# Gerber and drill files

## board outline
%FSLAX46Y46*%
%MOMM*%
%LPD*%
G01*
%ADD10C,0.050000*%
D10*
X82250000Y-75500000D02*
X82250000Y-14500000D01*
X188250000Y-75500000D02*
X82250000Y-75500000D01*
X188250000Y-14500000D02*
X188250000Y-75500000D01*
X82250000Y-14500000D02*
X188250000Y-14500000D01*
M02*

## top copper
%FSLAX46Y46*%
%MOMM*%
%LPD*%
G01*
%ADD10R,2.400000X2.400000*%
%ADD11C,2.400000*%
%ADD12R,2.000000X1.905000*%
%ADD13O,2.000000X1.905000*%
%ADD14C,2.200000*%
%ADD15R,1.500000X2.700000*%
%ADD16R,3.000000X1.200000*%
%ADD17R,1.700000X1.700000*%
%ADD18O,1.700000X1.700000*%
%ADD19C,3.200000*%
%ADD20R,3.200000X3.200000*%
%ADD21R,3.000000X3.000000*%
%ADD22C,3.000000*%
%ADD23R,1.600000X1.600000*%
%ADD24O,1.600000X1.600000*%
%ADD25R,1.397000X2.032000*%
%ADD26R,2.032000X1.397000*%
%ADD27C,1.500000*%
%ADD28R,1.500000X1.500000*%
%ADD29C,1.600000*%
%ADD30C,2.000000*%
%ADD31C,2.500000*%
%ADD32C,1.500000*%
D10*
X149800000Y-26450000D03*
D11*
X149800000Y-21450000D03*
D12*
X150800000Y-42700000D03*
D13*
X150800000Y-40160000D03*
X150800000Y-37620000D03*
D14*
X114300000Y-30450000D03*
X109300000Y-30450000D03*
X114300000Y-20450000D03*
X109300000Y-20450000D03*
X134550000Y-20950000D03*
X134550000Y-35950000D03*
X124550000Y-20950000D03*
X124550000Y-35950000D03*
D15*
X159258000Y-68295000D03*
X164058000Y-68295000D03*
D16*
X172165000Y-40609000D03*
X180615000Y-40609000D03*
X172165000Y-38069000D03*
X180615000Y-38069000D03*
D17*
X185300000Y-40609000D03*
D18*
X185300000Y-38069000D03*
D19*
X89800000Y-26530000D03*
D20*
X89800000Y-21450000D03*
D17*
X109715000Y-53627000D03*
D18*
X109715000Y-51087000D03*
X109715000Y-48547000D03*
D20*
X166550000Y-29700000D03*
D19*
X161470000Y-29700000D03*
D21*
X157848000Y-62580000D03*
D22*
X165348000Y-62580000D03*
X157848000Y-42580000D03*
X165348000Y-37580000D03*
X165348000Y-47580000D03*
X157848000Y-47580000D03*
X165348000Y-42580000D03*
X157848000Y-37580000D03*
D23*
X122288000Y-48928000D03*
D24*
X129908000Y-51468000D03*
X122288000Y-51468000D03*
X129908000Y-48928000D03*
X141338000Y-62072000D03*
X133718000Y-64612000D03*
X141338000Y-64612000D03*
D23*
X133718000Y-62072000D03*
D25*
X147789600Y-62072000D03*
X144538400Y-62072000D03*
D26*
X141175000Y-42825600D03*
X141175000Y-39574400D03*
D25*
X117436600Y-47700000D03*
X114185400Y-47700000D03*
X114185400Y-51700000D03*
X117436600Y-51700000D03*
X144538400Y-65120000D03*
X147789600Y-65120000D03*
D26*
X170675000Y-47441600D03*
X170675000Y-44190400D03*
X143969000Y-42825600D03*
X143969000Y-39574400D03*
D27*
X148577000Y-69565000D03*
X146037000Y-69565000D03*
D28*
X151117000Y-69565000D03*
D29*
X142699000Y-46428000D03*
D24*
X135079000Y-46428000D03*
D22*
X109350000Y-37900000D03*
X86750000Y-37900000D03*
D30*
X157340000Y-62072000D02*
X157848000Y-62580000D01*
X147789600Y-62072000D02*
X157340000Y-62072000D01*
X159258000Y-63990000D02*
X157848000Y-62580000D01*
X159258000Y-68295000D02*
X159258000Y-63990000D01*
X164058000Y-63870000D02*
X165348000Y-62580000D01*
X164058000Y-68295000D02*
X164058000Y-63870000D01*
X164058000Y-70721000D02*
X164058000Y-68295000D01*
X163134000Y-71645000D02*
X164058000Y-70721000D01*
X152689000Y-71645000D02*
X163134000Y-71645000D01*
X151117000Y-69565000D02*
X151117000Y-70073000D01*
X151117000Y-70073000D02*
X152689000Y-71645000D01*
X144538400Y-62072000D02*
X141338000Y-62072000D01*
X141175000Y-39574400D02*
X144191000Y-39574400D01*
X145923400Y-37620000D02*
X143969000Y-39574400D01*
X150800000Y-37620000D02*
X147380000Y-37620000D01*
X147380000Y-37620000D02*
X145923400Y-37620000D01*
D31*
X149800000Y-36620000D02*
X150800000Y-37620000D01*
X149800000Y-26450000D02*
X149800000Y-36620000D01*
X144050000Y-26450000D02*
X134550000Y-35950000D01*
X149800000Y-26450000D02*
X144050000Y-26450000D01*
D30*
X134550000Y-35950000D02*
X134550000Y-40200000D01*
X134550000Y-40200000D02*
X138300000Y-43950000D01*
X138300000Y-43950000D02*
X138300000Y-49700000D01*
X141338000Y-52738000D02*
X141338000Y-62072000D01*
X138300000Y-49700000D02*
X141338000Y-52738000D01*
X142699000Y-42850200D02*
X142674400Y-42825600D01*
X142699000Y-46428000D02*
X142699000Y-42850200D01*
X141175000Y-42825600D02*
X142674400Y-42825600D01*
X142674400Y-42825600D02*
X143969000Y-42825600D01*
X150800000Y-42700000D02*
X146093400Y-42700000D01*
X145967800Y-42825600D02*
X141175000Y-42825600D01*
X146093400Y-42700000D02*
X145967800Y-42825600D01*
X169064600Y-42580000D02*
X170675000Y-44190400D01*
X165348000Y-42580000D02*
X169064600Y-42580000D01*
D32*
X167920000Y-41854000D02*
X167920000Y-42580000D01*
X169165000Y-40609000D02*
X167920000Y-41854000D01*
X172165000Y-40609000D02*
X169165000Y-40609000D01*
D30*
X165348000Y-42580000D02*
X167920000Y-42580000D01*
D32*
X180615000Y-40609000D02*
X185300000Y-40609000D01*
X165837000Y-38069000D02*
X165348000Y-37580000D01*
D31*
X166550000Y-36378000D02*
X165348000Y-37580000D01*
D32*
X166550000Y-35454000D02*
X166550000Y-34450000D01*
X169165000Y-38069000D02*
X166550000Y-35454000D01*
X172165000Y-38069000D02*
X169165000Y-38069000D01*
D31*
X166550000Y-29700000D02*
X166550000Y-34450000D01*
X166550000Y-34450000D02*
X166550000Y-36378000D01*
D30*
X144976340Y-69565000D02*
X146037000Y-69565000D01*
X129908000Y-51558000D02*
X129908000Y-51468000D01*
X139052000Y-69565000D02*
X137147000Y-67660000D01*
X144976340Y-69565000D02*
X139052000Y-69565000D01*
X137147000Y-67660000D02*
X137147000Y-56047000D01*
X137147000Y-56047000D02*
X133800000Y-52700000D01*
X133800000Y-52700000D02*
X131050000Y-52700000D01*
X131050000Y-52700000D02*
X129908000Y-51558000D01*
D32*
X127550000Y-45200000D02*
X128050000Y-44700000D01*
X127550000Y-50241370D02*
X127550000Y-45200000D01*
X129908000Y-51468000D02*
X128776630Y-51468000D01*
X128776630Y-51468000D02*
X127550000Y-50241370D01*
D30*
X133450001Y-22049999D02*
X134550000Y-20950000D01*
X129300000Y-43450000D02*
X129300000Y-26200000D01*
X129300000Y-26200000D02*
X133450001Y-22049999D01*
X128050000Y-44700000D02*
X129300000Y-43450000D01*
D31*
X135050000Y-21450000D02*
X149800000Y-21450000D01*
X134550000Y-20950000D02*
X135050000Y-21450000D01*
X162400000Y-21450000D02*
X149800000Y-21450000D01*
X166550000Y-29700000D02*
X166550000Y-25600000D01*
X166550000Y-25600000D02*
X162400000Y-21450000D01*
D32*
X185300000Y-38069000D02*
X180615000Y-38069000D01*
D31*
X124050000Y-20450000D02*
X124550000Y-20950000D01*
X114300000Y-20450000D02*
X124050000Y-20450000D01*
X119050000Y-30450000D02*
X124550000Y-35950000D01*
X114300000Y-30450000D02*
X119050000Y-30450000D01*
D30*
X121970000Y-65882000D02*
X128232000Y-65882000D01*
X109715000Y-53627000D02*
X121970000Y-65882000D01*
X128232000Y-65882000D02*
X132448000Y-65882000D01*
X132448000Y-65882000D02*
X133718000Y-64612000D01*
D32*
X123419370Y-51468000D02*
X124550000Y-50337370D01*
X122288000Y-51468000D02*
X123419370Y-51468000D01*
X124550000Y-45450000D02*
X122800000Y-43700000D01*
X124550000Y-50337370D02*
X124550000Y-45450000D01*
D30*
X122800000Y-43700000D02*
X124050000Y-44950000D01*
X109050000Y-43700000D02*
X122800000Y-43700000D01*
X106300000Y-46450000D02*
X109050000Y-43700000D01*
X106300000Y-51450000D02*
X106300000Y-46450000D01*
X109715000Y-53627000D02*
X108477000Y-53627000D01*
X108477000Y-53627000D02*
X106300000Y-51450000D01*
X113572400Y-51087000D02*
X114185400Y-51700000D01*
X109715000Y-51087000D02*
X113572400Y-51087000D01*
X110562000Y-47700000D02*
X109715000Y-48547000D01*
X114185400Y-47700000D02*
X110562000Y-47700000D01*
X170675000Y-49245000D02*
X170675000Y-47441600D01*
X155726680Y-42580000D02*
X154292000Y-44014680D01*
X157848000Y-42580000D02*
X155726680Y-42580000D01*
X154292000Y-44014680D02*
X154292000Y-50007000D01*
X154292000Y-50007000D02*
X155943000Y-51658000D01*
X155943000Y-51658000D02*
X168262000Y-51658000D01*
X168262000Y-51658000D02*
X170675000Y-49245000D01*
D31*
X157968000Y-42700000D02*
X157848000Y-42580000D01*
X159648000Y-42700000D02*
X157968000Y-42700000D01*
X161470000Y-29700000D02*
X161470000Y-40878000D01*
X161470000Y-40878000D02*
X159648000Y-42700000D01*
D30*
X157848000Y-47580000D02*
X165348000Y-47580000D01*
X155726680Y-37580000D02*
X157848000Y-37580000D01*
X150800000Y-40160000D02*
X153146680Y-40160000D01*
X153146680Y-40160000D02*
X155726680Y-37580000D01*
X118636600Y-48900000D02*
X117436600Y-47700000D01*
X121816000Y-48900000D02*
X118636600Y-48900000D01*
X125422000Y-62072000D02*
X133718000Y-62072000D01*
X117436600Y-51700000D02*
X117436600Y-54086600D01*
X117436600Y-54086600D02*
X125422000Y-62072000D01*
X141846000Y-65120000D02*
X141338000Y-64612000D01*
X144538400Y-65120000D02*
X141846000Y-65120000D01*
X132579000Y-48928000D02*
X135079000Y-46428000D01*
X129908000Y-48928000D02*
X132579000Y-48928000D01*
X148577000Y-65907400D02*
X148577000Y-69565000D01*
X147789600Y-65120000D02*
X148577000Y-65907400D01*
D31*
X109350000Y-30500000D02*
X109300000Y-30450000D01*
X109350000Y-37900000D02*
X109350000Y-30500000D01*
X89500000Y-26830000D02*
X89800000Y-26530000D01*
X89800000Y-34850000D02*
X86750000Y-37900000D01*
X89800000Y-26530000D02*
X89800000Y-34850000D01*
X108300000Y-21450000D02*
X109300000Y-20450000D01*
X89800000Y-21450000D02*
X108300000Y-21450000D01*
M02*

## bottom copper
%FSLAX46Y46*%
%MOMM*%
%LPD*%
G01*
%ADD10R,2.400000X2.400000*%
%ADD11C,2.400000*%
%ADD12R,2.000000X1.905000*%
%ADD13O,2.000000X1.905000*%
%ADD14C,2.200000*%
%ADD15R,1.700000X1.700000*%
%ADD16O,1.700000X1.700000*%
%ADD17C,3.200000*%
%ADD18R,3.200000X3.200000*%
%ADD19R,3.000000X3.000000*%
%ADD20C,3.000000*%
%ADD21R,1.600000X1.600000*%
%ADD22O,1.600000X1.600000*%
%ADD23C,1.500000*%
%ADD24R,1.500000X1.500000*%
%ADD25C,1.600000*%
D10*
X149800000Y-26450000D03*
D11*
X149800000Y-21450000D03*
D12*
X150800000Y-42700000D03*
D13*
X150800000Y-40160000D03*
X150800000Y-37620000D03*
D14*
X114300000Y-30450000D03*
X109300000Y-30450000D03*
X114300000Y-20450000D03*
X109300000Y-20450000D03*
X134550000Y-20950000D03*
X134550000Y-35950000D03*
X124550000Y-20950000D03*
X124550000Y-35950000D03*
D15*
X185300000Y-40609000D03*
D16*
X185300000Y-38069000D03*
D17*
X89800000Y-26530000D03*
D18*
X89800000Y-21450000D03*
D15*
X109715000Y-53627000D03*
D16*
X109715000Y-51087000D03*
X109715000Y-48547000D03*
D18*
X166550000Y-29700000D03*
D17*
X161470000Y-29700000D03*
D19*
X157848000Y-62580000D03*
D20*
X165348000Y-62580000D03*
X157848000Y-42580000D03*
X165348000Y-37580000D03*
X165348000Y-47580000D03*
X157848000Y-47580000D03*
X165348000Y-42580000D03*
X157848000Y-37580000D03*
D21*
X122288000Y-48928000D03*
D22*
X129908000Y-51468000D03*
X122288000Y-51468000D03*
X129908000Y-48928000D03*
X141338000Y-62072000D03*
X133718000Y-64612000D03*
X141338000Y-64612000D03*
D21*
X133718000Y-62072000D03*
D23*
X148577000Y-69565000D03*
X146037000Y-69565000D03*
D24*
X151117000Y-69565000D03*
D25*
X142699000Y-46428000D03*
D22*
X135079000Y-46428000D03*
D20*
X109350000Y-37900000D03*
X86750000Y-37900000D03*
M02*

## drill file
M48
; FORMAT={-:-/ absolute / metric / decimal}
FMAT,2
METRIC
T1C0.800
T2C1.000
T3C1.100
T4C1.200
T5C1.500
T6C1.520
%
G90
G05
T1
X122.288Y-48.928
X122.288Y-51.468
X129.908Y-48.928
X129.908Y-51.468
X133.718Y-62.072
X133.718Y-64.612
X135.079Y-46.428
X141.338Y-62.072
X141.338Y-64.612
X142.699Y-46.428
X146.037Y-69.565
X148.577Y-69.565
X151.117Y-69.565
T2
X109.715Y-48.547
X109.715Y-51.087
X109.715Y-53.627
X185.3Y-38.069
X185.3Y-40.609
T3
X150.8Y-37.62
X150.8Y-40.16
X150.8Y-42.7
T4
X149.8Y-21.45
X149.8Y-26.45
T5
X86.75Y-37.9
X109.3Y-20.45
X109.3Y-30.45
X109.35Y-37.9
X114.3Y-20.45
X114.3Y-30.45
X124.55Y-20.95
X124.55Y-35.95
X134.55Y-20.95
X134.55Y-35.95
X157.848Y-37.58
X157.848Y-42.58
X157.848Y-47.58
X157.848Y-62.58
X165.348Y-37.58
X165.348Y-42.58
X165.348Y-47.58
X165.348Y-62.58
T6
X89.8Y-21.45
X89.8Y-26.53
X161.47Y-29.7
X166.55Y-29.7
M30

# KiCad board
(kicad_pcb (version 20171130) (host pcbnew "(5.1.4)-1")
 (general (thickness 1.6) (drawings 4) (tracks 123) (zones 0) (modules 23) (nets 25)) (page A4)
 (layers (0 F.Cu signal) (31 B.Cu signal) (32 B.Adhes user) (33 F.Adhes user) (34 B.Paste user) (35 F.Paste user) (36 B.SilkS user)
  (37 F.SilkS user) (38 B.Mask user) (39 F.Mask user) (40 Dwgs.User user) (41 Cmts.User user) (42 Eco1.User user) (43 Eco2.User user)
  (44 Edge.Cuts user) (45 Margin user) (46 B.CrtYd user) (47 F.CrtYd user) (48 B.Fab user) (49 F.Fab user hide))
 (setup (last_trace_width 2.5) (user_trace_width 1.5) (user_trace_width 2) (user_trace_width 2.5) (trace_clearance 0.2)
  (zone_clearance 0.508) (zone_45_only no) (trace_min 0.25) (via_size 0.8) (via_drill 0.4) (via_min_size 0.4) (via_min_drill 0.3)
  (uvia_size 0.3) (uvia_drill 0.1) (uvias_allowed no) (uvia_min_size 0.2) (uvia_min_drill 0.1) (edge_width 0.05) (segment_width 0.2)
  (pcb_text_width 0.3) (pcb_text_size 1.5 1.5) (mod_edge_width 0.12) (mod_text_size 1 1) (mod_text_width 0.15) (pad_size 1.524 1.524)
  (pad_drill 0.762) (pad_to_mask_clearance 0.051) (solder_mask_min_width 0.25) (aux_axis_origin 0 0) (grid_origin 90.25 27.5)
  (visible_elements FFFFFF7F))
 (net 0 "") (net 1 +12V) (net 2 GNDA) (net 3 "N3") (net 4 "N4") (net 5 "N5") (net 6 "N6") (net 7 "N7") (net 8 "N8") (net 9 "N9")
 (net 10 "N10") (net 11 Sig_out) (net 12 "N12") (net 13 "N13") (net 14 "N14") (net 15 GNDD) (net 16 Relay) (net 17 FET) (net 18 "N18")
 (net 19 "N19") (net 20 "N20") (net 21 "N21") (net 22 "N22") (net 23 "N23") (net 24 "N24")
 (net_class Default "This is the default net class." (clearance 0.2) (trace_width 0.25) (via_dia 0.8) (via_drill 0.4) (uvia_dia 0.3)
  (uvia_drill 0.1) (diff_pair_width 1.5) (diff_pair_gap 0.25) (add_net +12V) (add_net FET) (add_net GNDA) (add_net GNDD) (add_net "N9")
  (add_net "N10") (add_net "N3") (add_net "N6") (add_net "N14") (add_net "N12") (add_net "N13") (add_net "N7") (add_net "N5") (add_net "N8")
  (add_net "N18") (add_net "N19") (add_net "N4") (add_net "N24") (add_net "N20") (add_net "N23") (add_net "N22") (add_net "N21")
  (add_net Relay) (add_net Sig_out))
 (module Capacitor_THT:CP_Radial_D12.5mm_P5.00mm (layer F.Cu) (at 149.8 26.45 90)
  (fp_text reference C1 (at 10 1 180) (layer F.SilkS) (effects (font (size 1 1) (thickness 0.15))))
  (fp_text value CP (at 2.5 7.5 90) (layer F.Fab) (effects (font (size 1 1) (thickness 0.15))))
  (pad 1 thru_hole rect (at 0 0 90) (size 2.4 2.4) (drill 1.2) (layers *.Cu *.Mask) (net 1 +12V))
  (pad 2 thru_hole circle (at 5 0 90) (size 2.4 2.4) (drill 1.2) (layers *.Cu *.Mask) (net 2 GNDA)))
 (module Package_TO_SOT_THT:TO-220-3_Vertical (layer F.Cu) (at 150.8 42.7 90)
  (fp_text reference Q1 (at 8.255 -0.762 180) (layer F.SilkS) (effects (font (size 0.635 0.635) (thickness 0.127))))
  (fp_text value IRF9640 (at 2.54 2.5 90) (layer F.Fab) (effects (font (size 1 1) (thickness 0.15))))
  (pad 1 thru_hole rect (at 0 0 90) (size 1.905 2) (drill 1.1) (layers *.Cu *.Mask) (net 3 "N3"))
  (pad 2 thru_hole oval (at 2.54 0 90) (size 1.905 2) (drill 1.1) (layers *.Cu *.Mask) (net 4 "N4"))
  (pad 3 thru_hole oval (at 5.08 0 90) (size 1.905 2) (drill 1.1) (layers *.Cu *.Mask) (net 1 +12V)))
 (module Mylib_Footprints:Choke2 (layer F.Cu) (at 111.8 25.45)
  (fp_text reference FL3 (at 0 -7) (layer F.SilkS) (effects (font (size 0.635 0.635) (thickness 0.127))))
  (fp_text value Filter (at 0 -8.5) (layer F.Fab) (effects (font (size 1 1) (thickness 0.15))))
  (pad 3 thru_hole circle (at 2.5 5) (size 2.2 2.2) (drill 1.5) (layers *.Cu *.Mask) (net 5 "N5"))
  (pad 2 thru_hole circle (at -2.5 5) (size 2.2 2.2) (drill 1.5) (layers *.Cu *.Mask) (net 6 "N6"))
  (pad 4 thru_hole circle (at 2.5 -5) (size 2.2 2.2) (drill 1.5) (layers *.Cu *.Mask) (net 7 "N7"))
  (pad 1 thru_hole circle (at -2.5 -5) (size 2.2 2.2) (drill 1.5) (layers *.Cu *.Mask) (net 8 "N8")))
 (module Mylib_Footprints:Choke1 (layer F.Cu) (at 129.55 28.45)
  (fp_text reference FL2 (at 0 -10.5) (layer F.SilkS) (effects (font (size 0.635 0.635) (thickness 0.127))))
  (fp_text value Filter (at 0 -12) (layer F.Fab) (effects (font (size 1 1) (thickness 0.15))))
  (pad 4 thru_hole circle (at 5 -7.5) (size 2.2 2.2) (drill 1.5) (layers *.Cu *.Mask) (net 2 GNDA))
  (pad 3 thru_hole circle (at 5 7.5) (size 2.2 2.2) (drill 1.5) (layers *.Cu *.Mask) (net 1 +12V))
  (pad 1 thru_hole circle (at -5 -7.5) (size 2.2 2.2) (drill 1.5) (layers *.Cu *.Mask) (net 7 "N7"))
  (pad 2 thru_hole circle (at -5 7.5) (size 2.2 2.2) (drill 1.5) (layers *.Cu *.Mask) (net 5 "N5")))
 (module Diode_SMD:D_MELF (layer F.Cu) (at 161.658 68.295)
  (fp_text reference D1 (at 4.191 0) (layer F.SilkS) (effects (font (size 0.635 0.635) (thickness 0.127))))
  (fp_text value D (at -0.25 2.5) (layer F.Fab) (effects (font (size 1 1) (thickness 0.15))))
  (pad 1 smd rect (at -2.4 0) (size 1.5 2.7) (layers F.Cu F.Paste F.Mask) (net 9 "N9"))
  (pad 2 smd rect (at 2.4 0) (size 1.5 2.7) (layers F.Cu F.Paste F.Mask) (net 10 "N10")))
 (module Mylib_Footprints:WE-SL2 (layer F.Cu) (at 176.39 39.339)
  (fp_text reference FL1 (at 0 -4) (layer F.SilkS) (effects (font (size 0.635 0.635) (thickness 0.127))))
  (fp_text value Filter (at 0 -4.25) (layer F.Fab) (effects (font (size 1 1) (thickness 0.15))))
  (pad 2 smd rect (at -4.225 1.27) (size 3 1.2) (layers F.Cu F.Paste F.Mask) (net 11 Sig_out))
  (pad 3 smd rect (at 4.225 1.27) (size 3 1.2) (layers F.Cu F.Paste F.Mask) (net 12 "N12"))
  (pad 1 smd rect (at -4.225 -1.27) (size 3 1.2) (layers F.Cu F.Paste F.Mask) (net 2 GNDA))
  (pad 4 smd rect (at 4.225 -1.27) (size 3 1.2) (layers F.Cu F.Paste F.Mask) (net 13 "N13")))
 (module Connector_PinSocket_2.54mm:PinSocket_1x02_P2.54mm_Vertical (layer F.Cu) (at 185.3 40.609 180)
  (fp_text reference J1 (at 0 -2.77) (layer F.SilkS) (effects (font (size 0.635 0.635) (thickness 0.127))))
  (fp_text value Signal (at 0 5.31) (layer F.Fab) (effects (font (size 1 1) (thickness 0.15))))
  (pad 1 thru_hole rect (at 0 0 180) (size 1.7 1.7) (drill 1) (layers *.Cu *.Mask) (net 12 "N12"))
  (pad 2 thru_hole oval (at 0 2.54 180) (size 1.7 1.7) (drill 1) (layers *.Cu *.Mask) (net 13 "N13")))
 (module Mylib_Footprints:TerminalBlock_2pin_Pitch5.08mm (layer F.Cu) (at 89.8 21.45 270)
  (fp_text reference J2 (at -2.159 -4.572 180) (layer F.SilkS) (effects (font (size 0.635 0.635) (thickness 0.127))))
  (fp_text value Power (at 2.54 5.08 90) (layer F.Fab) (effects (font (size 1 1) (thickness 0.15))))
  (pad 2 thru_hole circle (at 5.08 0 270) (size 3.2 3.2) (drill 1.52) (layers *.Cu *.Mask) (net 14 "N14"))
  (pad 1 thru_hole rect (at 0 0 270) (size 3.2 3.2) (drill 1.52) (layers *.Cu *.Mask) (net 8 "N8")))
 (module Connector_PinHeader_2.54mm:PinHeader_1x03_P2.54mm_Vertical (layer F.Cu) (at 109.715 53.627 180)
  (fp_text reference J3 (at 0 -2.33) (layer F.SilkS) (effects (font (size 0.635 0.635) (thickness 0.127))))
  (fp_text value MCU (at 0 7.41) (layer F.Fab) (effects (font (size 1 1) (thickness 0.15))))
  (pad 1 thru_hole rect (at 0 0 180) (size 1.7 1.7) (drill 1) (layers *.Cu *.Mask) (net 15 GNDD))
  (pad 2 thru_hole oval (at 0 2.54 180) (size 1.7 1.7) (drill 1) (layers *.Cu *.Mask) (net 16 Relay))
  (pad 3 thru_hole oval (at 0 5.08 180) (size 1.7 1.7) (drill 1) (layers *.Cu *.Mask) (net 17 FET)))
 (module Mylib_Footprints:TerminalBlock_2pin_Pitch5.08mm (layer F.Cu) (at 166.55 29.7 180)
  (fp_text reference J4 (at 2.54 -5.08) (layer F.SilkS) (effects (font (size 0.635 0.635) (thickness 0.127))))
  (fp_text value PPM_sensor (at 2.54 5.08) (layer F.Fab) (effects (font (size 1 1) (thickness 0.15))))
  (pad 1 thru_hole rect (at 0 0 180) (size 3.2 3.2) (drill 1.52) (layers *.Cu *.Mask) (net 2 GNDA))
  (pad 2 thru_hole circle (at 5.08 0 180) (size 3.2 3.2) (drill 1.52) (layers *.Cu *.Mask) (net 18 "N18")))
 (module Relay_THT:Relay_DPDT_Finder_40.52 (layer F.Cu) (at 157.848 62.58 90)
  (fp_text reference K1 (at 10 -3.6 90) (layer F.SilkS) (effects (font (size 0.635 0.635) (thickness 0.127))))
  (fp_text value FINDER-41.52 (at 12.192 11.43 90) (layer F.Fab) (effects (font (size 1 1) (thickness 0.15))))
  (pad A1 thru_hole rect (at 0 0 90) (size 3 3) (drill 1.5) (layers *.Cu *.Mask) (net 9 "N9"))
  (pad A2 thru_hole circle (at 0 7.5 90) (size 3 3) (drill 1.5) (layers *.Cu *.Mask) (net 10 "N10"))
  (pad 11 thru_hole circle (at 20 0 90) (size 3 3) (drill 1.5) (layers *.Cu *.Mask) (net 18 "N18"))
  (pad 24 thru_hole circle (at 25 7.5 90) (size 3 3) (drill 1.5) (layers *.Cu *.Mask) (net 2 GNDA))
  (pad 22 thru_hole circle (at 15 7.5 90) (size 3 3) (drill 1.5) (layers *.Cu *.Mask) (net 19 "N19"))
  (pad 12 thru_hole circle (at 15 0 90) (size 3 3) (drill 1.5) (layers *.Cu *.Mask) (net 19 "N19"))
  (pad 21 thru_hole circle (at 20 7.5 90) (size 3 3) (drill 1.5) (layers *.Cu *.Mask) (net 11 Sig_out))
  (pad 14 thru_hole circle (at 25 0 90) (size 3 3) (drill 1.5) (layers *.Cu *.Mask) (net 4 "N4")))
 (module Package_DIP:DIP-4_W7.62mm (layer F.Cu) (at 122.288 48.928)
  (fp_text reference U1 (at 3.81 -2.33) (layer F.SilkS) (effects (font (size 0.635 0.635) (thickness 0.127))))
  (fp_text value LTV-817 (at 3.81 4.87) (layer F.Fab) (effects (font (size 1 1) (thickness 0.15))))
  (pad 1 thru_hole rect (at 0 0) (size 1.6 1.6) (drill 0.8) (layers *.Cu *.Mask) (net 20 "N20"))
  (pad 3 thru_hole oval (at 7.62 2.54) (size 1.6 1.6) (drill 0.8) (layers *.Cu *.Mask) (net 2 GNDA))
  (pad 2 thru_hole oval (at 0 2.54) (size 1.6 1.6) (drill 0.8) (layers *.Cu *.Mask) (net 15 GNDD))
  (pad 4 thru_hole oval (at 7.62 0) (size 1.6 1.6) (drill 0.8) (layers *.Cu *.Mask) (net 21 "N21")))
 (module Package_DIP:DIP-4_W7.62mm (layer F.Cu) (at 133.718 62.072)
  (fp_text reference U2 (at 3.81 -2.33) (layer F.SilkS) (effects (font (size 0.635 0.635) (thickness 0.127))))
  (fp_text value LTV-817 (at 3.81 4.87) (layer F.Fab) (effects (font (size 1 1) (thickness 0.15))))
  (pad 4 thru_hole oval (at 7.62 0) (size 1.6 1.6) (drill 0.8) (layers *.Cu *.Mask) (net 1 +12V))
  (pad 2 thru_hole oval (at 0 2.54) (size 1.6 1.6) (drill 0.8) (layers *.Cu *.Mask) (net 15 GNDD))
  (pad 3 thru_hole oval (at 7.62 2.54) (size 1.6 1.6) (drill 0.8) (layers *.Cu *.Mask) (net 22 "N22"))
  (pad 1 thru_hole rect (at 0 0) (size 1.6 1.6) (drill 0.8) (layers *.Cu *.Mask) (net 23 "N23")))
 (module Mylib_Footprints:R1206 (layer F.Cu) (at 146.164 62.072)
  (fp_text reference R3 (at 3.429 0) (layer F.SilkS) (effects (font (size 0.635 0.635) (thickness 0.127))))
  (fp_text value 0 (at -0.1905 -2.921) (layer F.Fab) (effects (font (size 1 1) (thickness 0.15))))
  (pad 2 smd rect (at 1.6256 0) (size 1.397 2.032) (layers F.Cu F.Paste F.Mask) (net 9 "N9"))
  (pad 1 smd rect (at -1.6256 0) (size 1.397 2.032) (layers F.Cu F.Paste F.Mask) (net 1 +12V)))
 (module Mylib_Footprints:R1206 (layer F.Cu) (at 141.175 41.2 270)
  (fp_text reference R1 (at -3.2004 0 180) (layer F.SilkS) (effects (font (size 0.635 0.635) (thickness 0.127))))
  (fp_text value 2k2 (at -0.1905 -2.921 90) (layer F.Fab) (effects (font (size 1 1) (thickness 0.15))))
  (pad 2 smd rect (at 1.6256 0 270) (size 1.397 2.032) (layers F.Cu F.Paste F.Mask) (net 3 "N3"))
  (pad 1 smd rect (at -1.6256 0 270) (size 1.397 2.032) (layers F.Cu F.Paste F.Mask) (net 1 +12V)))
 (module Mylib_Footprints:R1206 (layer F.Cu) (at 115.811 47.7 180)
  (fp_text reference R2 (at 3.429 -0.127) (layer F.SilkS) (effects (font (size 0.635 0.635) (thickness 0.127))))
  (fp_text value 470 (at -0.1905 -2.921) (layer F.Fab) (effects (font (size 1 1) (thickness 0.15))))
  (pad 1 smd rect (at -1.6256 0 180) (size 1.397 2.032) (layers F.Cu F.Paste F.Mask) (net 20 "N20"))
  (pad 2 smd rect (at 1.6256 0 180) (size 1.397 2.032) (layers F.Cu F.Paste F.Mask) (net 17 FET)))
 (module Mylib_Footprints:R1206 (layer F.Cu) (at 115.811 51.7 180)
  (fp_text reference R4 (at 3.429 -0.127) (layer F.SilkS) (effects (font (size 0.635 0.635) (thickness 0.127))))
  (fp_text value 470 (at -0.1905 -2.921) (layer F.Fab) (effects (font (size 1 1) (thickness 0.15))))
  (pad 2 smd rect (at 1.6256 0 180) (size 1.397 2.032) (layers F.Cu F.Paste F.Mask) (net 16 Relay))
  (pad 1 smd rect (at -1.6256 0 180) (size 1.397 2.032) (layers F.Cu F.Paste F.Mask) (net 23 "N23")))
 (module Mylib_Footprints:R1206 (layer F.Cu) (at 146.164 65.12)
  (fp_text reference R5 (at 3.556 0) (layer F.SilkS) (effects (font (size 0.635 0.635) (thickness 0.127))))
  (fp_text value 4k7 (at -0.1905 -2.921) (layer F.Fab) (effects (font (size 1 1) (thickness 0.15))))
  (pad 1 smd rect (at -1.6256 0) (size 1.397 2.032) (layers F.Cu F.Paste F.Mask) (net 22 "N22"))
  (pad 2 smd rect (at 1.6256 0) (size 1.397 2.032) (layers F.Cu F.Paste F.Mask) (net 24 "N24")))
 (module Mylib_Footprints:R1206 (layer F.Cu) (at 170.675 45.816 270)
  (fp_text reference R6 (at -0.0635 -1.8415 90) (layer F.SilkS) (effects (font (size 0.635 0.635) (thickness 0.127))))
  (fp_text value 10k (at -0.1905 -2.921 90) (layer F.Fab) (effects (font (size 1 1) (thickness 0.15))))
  (pad 2 smd rect (at 1.6256 0 270) (size 1.397 2.032) (layers F.Cu F.Paste F.Mask) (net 18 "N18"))
  (pad 1 smd rect (at -1.6256 0 270) (size 1.397 2.032) (layers F.Cu F.Paste F.Mask) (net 11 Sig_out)))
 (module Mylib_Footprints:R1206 (layer F.Cu) (at 143.969 41.2 270)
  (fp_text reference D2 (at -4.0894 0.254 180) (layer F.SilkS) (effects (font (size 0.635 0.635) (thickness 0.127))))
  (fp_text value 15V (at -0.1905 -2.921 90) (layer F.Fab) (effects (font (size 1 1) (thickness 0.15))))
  (pad 2 smd rect (at 1.6256 0 270) (size 1.397 2.032) (layers F.Cu F.Paste F.Mask) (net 3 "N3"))
  (pad 1 smd rect (at -1.6256 0 270) (size 1.397 2.032) (layers F.Cu F.Paste F.Mask) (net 1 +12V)))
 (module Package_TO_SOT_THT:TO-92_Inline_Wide (layer F.Cu) (at 151.117 69.565 180)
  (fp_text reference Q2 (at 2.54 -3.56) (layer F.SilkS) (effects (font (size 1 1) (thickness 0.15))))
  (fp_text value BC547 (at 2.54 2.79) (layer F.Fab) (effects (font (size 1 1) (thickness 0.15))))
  (pad 2 thru_hole circle (at 2.54 0 270) (size 1.5 1.5) (drill 0.8) (layers *.Cu *.Mask) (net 24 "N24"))
  (pad 3 thru_hole circle (at 5.08 0 270) (size 1.5 1.5) (drill 0.8) (layers *.Cu *.Mask) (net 2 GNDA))
  (pad 1 thru_hole rect (at 0 0 270) (size 1.5 1.5) (drill 0.8) (layers *.Cu *.Mask) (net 10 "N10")))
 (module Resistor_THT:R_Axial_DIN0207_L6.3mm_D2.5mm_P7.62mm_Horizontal (layer F.Cu) (at 142.699 46.428 180)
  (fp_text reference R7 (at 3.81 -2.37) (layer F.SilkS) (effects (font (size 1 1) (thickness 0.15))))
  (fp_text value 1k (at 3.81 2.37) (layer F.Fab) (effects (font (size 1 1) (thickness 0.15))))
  (pad 1 thru_hole circle (at 0 0 180) (size 1.6 1.6) (drill 0.8) (layers *.Cu *.Mask) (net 3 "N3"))
  (pad 2 thru_hole oval (at 7.62 0 180) (size 1.6 1.6) (drill 0.8) (layers *.Cu *.Mask) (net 21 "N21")))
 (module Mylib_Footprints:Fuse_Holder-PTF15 (layer F.Cu) (at 98.05 37.9 180)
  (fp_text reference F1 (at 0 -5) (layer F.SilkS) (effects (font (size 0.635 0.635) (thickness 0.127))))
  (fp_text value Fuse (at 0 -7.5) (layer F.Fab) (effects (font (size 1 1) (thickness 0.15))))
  (pad 1 thru_hole circle (at -11.3 0 180) (size 3 3) (drill 1.5) (layers *.Cu *.Mask) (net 6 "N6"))
  (pad 2 thru_hole circle (at 11.3 0 180) (size 3 3) (drill 1.5) (layers *.Cu *.Mask) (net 14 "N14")))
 (gr_line (start 82.25 75.5) (end 82.25 14.5) (layer Edge.Cuts) (width 0.05))
 (gr_line (start 188.25 75.5) (end 82.25 75.5) (layer Edge.Cuts) (width 0.05))
 (gr_line (start 188.25 14.5) (end 188.25 75.5) (layer Edge.Cuts) (width 0.05))
 (gr_line (start 82.25 14.5) (end 188.25 14.5) (layer Edge.Cuts) (width 0.05))
 (segment (start 157.34 62.072) (end 157.848 62.58) (width 2) (layer F.Cu) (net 9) (status 30))
 (segment (start 147.7896 62.072) (end 157.34 62.072) (width 2) (layer F.Cu) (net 9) (status 30))
 (segment (start 159.258 63.99) (end 157.848 62.58) (width 2) (layer F.Cu) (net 9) (status 30))
 (segment (start 159.258 68.295) (end 159.258 63.99) (width 2) (layer F.Cu) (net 9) (status 30))
 (segment (start 164.058 63.87) (end 165.348 62.58) (width 2) (layer F.Cu) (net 10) (status 20))
 (segment (start 164.058 68.295) (end 164.058 63.87) (width 2) (layer F.Cu) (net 10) (status 10))
 (segment (start 164.058 70.721) (end 164.058 68.295) (width 2) (layer F.Cu) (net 10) (status 20))
 (segment (start 163.134 71.645) (end 164.058 70.721) (width 2) (layer F.Cu) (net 10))
 (segment (start 152.689 71.645) (end 163.134 71.645) (width 2) (layer F.Cu) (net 10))
 (segment (start 151.117 69.565) (end 151.117 70.073) (width 2) (layer F.Cu) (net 10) (status 30))
 (segment (start 151.117 70.073) (end 152.689 71.645) (width 2) (layer F.Cu) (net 10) (status 10))
 (segment (start 144.5384 62.072) (end 141.338 62.072) (width 2) (layer F.Cu) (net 1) (status 30))
 (segment (start 141.175 39.5744) (end 144.191 39.5744) (width 2) (layer F.Cu) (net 1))
 (segment (start 145.9234 37.62) (end 143.969 39.5744) (width 2) (layer F.Cu) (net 1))
 (segment (start 150.8 37.62) (end 147.38 37.62) (width 2) (layer F.Cu) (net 1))
 (segment (start 147.38 37.62) (end 145.9234 37.62) (width 2) (layer F.Cu) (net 1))
 (segment (start 149.8 36.62) (end 150.8 37.62) (width 2.5) (layer F.Cu) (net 1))
 (segment (start 149.8 26.45) (end 149.8 36.62) (width 2.5) (layer F.Cu) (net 1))
 (segment (start 144.05 26.45) (end 134.55 35.95) (width 2.5) (layer F.Cu) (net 1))
 (segment (start 149.8 26.45) (end 144.05 26.45) (width 2.5) (layer F.Cu) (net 1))
 (segment (start 134.55 35.95) (end 134.55 40.2) (width 2) (layer F.Cu) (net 1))
 (segment (start 134.55 40.2) (end 138.3 43.95) (width 2) (layer F.Cu) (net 1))
 (segment (start 138.3 43.95) (end 138.3 49.7) (width 2) (layer F.Cu) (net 1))
 (segment (start 141.338 52.738) (end 141.338 62.072) (width 2) (layer F.Cu) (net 1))
 (segment (start 138.3 49.7) (end 141.338 52.738) (width 2) (layer F.Cu) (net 1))
 (segment (start 142.699 42.8502) (end 142.6744 42.8256) (width 2) (layer F.Cu) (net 3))
 (segment (start 142.699 46.428) (end 142.699 42.8502) (width 2) (layer F.Cu) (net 3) (status 10))
 (segment (start 141.175 42.8256) (end 142.6744 42.8256) (width 2) (layer F.Cu) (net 3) (status 10))
 (segment (start 142.6744 42.8256) (end 143.969 42.8256) (width 2) (layer F.Cu) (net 3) (status 20))
 (segment (start 150.8 42.7) (end 146.0934 42.7) (width 2) (layer F.Cu) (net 3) (status 10))
 (segment (start 145.9678 42.8256) (end 141.175 42.8256) (width 2) (layer F.Cu) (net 3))
 (segment (start 146.0934 42.7) (end 145.9678 42.8256) (width 2) (layer F.Cu) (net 3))
 (segment (start 169.0646 42.58) (end 170.675 44.1904) (width 2) (layer F.Cu) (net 11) (status 20))
 (segment (start 165.348 42.58) (end 169.0646 42.58) (width 2) (layer F.Cu) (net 11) (status 10))
 (segment (start 167.92 41.854) (end 167.92 42.58) (width 1.5) (layer F.Cu) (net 11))
 (segment (start 169.165 40.609) (end 167.92 41.854) (width 1.5) (layer F.Cu) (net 11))
 (segment (start 172.165 40.609) (end 169.165 40.609) (width 1.5) (layer F.Cu) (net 11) (status 10))
 (segment (start 165.348 42.58) (end 167.92 42.58) (width 2) (layer F.Cu) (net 11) (status 10))
 (segment (start 180.615 40.609) (end 185.3 40.609) (width 1.5) (layer F.Cu) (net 12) (status 30))
 (segment (start 165.837 38.069) (end 165.348 37.58) (width 1.5) (layer F.Cu) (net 2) (status 30))
 (segment (start 166.55 36.378) (end 165.348 37.58) (width 2.5) (layer F.Cu) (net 2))
 (segment (start 166.55 35.454) (end 166.55 34.45) (width 1.5) (layer F.Cu) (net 2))
 (segment (start 169.165 38.069) (end 166.55 35.454) (width 1.5) (layer F.Cu) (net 2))
 (segment (start 172.165 38.069) (end 169.165 38.069) (width 1.5) (layer F.Cu) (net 2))
 (segment (start 166.55 29.7) (end 166.55 34.45) (width 2.5) (layer F.Cu) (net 2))
 (segment (start 166.55 34.45) (end 166.55 36.378) (width 2.5) (layer F.Cu) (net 2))
 (segment (start 144.97634 69.565) (end 146.037 69.565) (width 2) (layer F.Cu) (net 2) (status 20))
 (segment (start 129.908 51.558) (end 129.908 51.468) (width 2) (layer F.Cu) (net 2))
 (segment (start 139.052 69.565) (end 137.147 67.66) (width 2) (layer F.Cu) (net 2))
 (segment (start 144.97634 69.565) (end 139.052 69.565) (width 2) (layer F.Cu) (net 2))
 (segment (start 137.147 67.66) (end 137.147 56.047) (width 2) (layer F.Cu) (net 2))
 (segment (start 137.147 56.047) (end 133.8 52.7) (width 2) (layer F.Cu) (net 2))
 (segment (start 133.8 52.7) (end 131.05 52.7) (width 2) (layer F.Cu) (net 2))
 (segment (start 131.05 52.7) (end 129.908 51.558) (width 2) (layer F.Cu) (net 2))
 (segment (start 127.55 45.2) (end 128.05 44.7) (width 1.5) (layer F.Cu) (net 2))
 (segment (start 127.55 50.24137) (end 127.55 45.2) (width 1.5) (layer F.Cu) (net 2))
 (segment (start 129.908 51.468) (end 128.77663 51.468) (width 1.5) (layer F.Cu) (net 2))
 (segment (start 128.77663 51.468) (end 127.55 50.24137) (width 1.5) (layer F.Cu) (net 2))
 (segment (start 133.450001 22.049999) (end 134.55 20.95) (width 2) (layer F.Cu) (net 2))
 (segment (start 129.3 43.45) (end 129.3 26.2) (width 2) (layer F.Cu) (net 2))
 (segment (start 129.3 26.2) (end 133.450001 22.049999) (width 2) (layer F.Cu) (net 2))
 (segment (start 128.05 44.7) (end 129.3 43.45) (width 2) (layer F.Cu) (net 2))
 (segment (start 135.05 21.45) (end 149.8 21.45) (width 2.5) (layer F.Cu) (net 2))
 (segment (start 134.55 20.95) (end 135.05 21.45) (width 2.5) (layer F.Cu) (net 2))
 (segment (start 162.4 21.45) (end 149.8 21.45) (width 2.5) (layer F.Cu) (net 2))
 (segment (start 166.55 29.7) (end 166.55 25.6) (width 2.5) (layer F.Cu) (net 2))
 (segment (start 166.55 25.6) (end 162.4 21.45) (width 2.5) (layer F.Cu) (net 2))
 (segment (start 185.3 38.069) (end 180.615 38.069) (width 1.5) (layer F.Cu) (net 13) (status 30))
 (segment (start 124.05 20.45) (end 124.55 20.95) (width 2.5) (layer F.Cu) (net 7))
 (segment (start 114.3 20.45) (end 124.05 20.45) (width 2.5) (layer F.Cu) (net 7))
 (segment (start 119.05 30.45) (end 124.55 35.95) (width 2.5) (layer F.Cu) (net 5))
 (segment (start 114.3 30.45) (end 119.05 30.45) (width 2.5) (layer F.Cu) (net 5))
 (segment (start 121.97 65.882) (end 128.232 65.882) (width 2) (layer F.Cu) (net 15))
 (segment (start 109.715 53.627) (end 121.97 65.882) (width 2) (layer F.Cu) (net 15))
 (segment (start 128.232 65.882) (end 132.448 65.882) (width 2) (layer F.Cu) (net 15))
 (segment (start 132.448 65.882) (end 133.718 64.612) (width 2) (layer F.Cu) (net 15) (status 20))
 (segment (start 123.41937 51.468) (end 124.55 50.33737) (width 1.5) (layer F.Cu) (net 15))
 (segment (start 122.288 51.468) (end 123.41937 51.468) (width 1.5) (layer F.Cu) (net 15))
 (segment (start 124.55 45.45) (end 122.8 43.7) (width 1.5) (layer F.Cu) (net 15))
 (segment (start 124.55 50.33737) (end 124.55 45.45) (width 1.5) (layer F.Cu) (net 15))
 (segment (start 122.8 43.7) (end 124.05 44.95) (width 2) (layer F.Cu) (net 15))
 (segment (start 109.05 43.7) (end 122.8 43.7) (width 2) (layer F.Cu) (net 15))
 (segment (start 106.3 46.45) (end 109.05 43.7) (width 2) (layer F.Cu) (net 15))
 (segment (start 106.3 51.45) (end 106.3 46.45) (width 2) (layer F.Cu) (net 15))
 (segment (start 109.715 53.627) (end 108.477 53.627) (width 2) (layer F.Cu) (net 15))
 (segment (start 108.477 53.627) (end 106.3 51.45) (width 2) (layer F.Cu) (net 15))
 (segment (start 113.5724 51.087) (end 114.1854 51.7) (width 2) (layer F.Cu) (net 16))
 (segment (start 109.715 51.087) (end 113.5724 51.087) (width 2) (layer F.Cu) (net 16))
 (segment (start 110.562 47.7) (end 109.715 48.547) (width 2) (layer F.Cu) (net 17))
 (segment (start 114.1854 47.7) (end 110.562 47.7) (width 2) (layer F.Cu) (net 17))
 (segment (start 170.675 49.245) (end 170.675 47.4416) (width 2) (layer F.Cu) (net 18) (status 20))
 (segment (start 155.72668 42.58) (end 154.292 44.01468) (width 2) (layer F.Cu) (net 18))
 (segment (start 157.848 42.58) (end 155.72668 42.58) (width 2) (layer F.Cu) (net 18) (status 10))
 (segment (start 154.292 44.01468) (end 154.292 50.007) (width 2) (layer F.Cu) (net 18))
 (segment (start 154.292 50.007) (end 155.943 51.658) (width 2) (layer F.Cu) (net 18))
 (segment (start 155.943 51.658) (end 168.262 51.658) (width 2) (layer F.Cu) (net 18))
 (segment (start 168.262 51.658) (end 170.675 49.245) (width 2) (layer F.Cu) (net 18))
 (segment (start 157.968 42.7) (end 157.848 42.58) (width 2.5) (layer F.Cu) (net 18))
 (segment (start 159.648 42.7) (end 157.968 42.7) (width 2.5) (layer F.Cu) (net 18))
 (segment (start 161.47 29.7) (end 161.47 40.878) (width 2.5) (layer F.Cu) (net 18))
 (segment (start 161.47 40.878) (end 159.648 42.7) (width 2.5) (layer F.Cu) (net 18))
 (segment (start 157.848 47.58) (end 165.348 47.58) (width 2) (layer F.Cu) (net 19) (status 30))
 (segment (start 155.72668 37.58) (end 157.848 37.58) (width 2) (layer F.Cu) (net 4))
 (segment (start 150.8 40.16) (end 153.14668 40.16) (width 2) (layer F.Cu) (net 4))
 (segment (start 153.14668 40.16) (end 155.72668 37.58) (width 2) (layer F.Cu) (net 4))
 (segment (start 118.6366 48.9) (end 117.4366 47.7) (width 2) (layer F.Cu) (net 20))
 (segment (start 121.816 48.9) (end 118.6366 48.9) (width 2) (layer F.Cu) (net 20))
 (segment (start 125.422 62.072) (end 133.718 62.072) (width 2) (layer F.Cu) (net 23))
 (segment (start 117.4366 51.7) (end 117.4366 54.0866) (width 2) (layer F.Cu) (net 23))
 (segment (start 117.4366 54.0866) (end 125.422 62.072) (width 2) (layer F.Cu) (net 23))
 (segment (start 141.846 65.12) (end 141.338 64.612) (width 2) (layer F.Cu) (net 22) (status 30))
 (segment (start 144.5384 65.12) (end 141.846 65.12) (width 2) (layer F.Cu) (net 22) (status 30))
 (segment (start 132.579 48.928) (end 135.079 46.428) (width 2) (layer F.Cu) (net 21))
 (segment (start 129.908 48.928) (end 132.579 48.928) (width 2) (layer F.Cu) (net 21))
 (segment (start 148.577 65.9074) (end 148.577 69.565) (width 2) (layer F.Cu) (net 24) (status 20))
 (segment (start 147.7896 65.12) (end 148.577 65.9074) (width 2) (layer F.Cu) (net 24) (status 10))
 (segment (start 109.35 30.5) (end 109.3 30.45) (width 2.5) (layer F.Cu) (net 6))
 (segment (start 109.35 37.9) (end 109.35 30.5) (width 2.5) (layer F.Cu) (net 6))
 (segment (start 89.5 26.83) (end 89.8 26.53) (width 2.5) (layer F.Cu) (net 14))
 (segment (start 89.8 34.85) (end 86.75 37.9) (width 2.5) (layer F.Cu) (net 14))
 (segment (start 89.8 26.53) (end 89.8 34.85) (width 2.5) (layer F.Cu) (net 14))
 (segment (start 108.3 21.45) (end 109.3 20.45) (width 2.5) (layer F.Cu) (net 8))
 (segment (start 89.8 21.45) (end 108.3 21.45) (width 2.5) (layer F.Cu) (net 8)))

